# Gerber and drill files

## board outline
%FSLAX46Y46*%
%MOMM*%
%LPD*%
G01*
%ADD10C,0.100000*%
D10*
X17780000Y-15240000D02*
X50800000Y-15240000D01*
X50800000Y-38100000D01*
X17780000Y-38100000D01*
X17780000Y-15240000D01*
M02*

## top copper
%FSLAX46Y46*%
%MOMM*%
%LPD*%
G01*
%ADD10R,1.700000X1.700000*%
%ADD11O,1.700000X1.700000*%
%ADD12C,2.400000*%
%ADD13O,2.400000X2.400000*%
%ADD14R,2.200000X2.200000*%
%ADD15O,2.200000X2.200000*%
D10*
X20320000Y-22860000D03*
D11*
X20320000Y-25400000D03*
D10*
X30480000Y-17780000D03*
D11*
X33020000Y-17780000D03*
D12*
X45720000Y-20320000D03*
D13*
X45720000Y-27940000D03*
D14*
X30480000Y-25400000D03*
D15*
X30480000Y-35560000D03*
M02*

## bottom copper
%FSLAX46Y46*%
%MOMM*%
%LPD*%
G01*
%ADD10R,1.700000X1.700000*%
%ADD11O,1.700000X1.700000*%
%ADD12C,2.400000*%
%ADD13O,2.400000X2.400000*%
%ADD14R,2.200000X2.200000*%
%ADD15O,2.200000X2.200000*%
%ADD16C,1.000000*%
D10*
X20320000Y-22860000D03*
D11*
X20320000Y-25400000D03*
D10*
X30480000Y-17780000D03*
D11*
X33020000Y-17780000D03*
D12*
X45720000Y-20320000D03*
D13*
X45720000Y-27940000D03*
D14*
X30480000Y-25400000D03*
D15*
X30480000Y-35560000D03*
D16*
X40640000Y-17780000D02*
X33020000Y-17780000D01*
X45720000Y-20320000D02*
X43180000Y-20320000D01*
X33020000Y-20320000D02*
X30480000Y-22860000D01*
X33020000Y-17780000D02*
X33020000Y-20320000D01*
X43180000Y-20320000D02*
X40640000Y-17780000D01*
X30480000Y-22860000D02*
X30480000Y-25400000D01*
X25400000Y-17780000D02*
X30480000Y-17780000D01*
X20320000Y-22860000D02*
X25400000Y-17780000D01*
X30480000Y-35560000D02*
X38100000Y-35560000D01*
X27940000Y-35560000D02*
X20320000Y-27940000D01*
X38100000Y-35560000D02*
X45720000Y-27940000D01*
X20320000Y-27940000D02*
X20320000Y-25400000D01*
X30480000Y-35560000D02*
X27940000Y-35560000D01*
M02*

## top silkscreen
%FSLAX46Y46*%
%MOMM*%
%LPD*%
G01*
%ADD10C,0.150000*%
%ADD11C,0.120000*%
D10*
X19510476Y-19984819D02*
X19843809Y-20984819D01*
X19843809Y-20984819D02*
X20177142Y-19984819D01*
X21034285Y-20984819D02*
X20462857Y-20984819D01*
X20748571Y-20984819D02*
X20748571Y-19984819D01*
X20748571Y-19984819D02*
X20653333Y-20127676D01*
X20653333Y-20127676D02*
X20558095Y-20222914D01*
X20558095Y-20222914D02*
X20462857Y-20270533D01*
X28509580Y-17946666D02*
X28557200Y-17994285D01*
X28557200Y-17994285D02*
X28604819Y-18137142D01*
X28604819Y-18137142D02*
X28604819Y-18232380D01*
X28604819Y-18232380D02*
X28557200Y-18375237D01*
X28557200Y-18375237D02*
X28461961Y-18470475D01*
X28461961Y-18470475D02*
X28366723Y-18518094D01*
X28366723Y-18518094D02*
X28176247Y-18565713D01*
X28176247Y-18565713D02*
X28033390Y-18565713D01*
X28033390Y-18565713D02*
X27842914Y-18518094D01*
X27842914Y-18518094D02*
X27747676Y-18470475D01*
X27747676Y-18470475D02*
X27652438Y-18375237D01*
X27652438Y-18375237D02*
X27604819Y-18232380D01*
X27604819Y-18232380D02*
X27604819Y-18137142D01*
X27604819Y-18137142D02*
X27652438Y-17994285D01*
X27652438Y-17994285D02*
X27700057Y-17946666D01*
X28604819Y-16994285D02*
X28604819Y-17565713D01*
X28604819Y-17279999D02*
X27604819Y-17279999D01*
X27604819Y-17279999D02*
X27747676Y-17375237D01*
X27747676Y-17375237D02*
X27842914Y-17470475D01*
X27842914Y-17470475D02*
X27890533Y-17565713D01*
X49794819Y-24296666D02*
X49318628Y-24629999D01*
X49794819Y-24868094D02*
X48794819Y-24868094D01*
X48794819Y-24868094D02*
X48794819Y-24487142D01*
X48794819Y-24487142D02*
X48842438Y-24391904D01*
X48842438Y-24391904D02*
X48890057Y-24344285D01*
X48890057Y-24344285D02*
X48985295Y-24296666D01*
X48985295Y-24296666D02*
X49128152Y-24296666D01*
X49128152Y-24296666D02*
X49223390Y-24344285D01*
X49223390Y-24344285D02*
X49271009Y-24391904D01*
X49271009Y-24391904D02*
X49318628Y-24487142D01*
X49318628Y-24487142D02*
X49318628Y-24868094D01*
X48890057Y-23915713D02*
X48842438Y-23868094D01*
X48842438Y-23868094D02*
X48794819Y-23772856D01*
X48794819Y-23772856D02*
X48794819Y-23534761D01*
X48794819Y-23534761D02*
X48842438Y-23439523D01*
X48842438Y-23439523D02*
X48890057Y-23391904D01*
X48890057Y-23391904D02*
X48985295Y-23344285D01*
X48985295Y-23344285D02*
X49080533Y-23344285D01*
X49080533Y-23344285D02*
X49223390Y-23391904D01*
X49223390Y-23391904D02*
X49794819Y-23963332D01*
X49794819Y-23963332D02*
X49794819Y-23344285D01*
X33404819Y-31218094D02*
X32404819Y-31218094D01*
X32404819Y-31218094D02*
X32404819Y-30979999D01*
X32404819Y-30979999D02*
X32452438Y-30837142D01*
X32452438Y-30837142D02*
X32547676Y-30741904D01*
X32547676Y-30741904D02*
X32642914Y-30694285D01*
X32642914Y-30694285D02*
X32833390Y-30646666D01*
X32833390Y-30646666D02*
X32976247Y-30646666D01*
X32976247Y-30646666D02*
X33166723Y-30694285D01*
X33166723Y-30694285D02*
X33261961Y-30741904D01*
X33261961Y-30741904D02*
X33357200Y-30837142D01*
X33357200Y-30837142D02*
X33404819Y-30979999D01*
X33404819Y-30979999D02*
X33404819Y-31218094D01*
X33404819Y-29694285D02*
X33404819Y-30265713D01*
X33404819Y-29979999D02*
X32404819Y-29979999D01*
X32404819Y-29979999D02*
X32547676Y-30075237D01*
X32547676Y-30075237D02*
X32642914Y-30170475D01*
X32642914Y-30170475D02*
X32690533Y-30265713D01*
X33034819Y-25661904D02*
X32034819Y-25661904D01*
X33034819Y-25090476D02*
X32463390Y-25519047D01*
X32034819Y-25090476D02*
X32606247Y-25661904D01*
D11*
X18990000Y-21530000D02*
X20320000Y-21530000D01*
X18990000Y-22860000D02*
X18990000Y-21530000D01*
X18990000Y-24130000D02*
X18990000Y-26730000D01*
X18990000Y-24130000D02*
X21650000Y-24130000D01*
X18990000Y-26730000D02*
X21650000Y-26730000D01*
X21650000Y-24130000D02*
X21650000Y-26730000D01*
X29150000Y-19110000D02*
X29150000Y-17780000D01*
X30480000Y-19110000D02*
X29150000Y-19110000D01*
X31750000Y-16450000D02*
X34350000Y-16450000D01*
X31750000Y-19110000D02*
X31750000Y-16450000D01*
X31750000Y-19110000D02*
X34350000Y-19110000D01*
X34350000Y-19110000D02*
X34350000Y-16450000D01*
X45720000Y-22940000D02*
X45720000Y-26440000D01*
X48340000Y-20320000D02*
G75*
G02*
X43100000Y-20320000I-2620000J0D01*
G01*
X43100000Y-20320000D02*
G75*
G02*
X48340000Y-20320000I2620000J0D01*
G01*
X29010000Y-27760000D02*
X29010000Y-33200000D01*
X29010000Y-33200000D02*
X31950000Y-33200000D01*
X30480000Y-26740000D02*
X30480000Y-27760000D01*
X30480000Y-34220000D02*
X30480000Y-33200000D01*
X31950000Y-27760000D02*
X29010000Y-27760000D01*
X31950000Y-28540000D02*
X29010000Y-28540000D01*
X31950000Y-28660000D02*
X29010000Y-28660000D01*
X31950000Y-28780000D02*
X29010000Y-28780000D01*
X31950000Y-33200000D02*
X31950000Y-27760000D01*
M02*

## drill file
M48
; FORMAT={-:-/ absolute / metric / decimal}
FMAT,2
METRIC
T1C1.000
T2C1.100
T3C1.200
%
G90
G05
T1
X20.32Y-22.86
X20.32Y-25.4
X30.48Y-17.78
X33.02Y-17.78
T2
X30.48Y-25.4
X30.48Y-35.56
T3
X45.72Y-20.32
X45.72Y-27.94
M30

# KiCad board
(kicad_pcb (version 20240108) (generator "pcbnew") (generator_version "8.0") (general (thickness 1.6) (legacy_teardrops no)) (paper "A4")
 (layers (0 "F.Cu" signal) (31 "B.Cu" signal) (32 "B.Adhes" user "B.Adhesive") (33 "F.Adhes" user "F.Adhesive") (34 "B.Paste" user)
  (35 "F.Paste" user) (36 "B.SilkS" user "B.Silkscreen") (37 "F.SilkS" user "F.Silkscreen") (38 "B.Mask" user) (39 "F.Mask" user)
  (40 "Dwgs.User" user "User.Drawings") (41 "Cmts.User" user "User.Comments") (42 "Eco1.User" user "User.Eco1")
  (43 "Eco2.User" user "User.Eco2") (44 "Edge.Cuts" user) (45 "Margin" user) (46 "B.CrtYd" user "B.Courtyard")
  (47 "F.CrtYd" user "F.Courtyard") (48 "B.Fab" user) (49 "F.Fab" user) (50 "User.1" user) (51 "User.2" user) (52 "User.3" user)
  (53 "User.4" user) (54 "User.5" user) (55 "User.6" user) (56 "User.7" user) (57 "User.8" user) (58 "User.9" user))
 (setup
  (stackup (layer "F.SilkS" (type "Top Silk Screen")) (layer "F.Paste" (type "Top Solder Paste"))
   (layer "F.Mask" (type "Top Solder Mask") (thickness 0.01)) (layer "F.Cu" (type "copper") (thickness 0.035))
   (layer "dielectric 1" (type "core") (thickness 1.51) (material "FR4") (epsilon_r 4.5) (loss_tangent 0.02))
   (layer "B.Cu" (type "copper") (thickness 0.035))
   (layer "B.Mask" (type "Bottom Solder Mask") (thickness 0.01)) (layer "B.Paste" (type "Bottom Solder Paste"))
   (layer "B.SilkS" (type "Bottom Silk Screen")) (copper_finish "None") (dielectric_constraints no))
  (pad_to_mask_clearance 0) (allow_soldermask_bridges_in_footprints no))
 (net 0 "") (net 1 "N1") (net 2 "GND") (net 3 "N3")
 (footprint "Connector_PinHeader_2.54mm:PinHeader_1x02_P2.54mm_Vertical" (layer "F.Cu") (at 20.32 22.86)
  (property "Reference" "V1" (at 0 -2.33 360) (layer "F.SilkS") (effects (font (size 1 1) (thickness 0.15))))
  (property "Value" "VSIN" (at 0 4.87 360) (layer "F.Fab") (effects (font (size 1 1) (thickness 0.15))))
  (fp_line (start -1.33 -1.33) (end 0 -1.33) (stroke (width 0.12) (type solid)) (layer "F.SilkS"))
  (fp_line (start -1.33 0) (end -1.33 -1.33) (stroke (width 0.12) (type solid)) (layer "F.SilkS"))
  (fp_line (start -1.33 1.27) (end -1.33 3.87) (stroke (width 0.12) (type solid)) (layer "F.SilkS"))
  (fp_line (start -1.33 1.27) (end 1.33 1.27) (stroke (width 0.12) (type solid)) (layer "F.SilkS"))
  (fp_line (start -1.33 3.87) (end 1.33 3.87) (stroke (width 0.12) (type solid)) (layer "F.SilkS"))
  (fp_line (start 1.33 1.27) (end 1.33 3.87) (stroke (width 0.12) (type solid)) (layer "F.SilkS"))
  (pad "1" thru_hole rect (at 0 0) (size 1.7 1.7) (drill 1) (layers "*.Cu" "*.Mask") (remove_unused_layers no) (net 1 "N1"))
  (pad "2" thru_hole oval (at 0 2.54) (size 1.7 1.7) (drill 1) (layers "*.Cu" "*.Mask") (remove_unused_layers no) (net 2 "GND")))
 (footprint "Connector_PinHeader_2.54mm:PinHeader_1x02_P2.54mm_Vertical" (layer "F.Cu") (at 30.48 17.78 90)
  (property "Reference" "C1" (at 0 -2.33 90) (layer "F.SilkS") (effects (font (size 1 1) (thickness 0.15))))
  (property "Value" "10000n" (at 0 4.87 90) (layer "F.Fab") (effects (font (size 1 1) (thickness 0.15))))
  (fp_line (start -1.33 -1.33) (end 0 -1.33) (stroke (width 0.12) (type solid)) (layer "F.SilkS"))
  (fp_line (start -1.33 0) (end -1.33 -1.33) (stroke (width 0.12) (type solid)) (layer "F.SilkS"))
  (fp_line (start 1.33 1.27) (end 1.33 3.87) (stroke (width 0.12) (type solid)) (layer "F.SilkS"))
  (fp_line (start -1.33 1.27) (end 1.33 1.27) (stroke (width 0.12) (type solid)) (layer "F.SilkS"))
  (fp_line (start -1.33 1.27) (end -1.33 3.87) (stroke (width 0.12) (type solid)) (layer "F.SilkS"))
  (fp_line (start -1.33 3.87) (end 1.33 3.87) (stroke (width 0.12) (type solid)) (layer "F.SilkS"))
  (pad "1" thru_hole rect (at 0 0 90) (size 1.7 1.7) (drill 1) (layers "*.Cu" "*.Mask") (remove_unused_layers no) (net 1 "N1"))
  (pad "2" thru_hole oval (at 0 2.54 90) (size 1.7 1.7) (drill 1) (layers "*.Cu" "*.Mask") (remove_unused_layers no) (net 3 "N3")))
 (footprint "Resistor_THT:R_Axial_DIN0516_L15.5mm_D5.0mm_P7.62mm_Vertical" (layer "F.Cu") (at 45.72 20.32 -90)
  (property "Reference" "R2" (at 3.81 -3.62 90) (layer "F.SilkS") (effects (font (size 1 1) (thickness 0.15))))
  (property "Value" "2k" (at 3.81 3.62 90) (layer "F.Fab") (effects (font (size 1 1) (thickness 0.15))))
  (fp_line (start 2.62 0) (end 6.12 0) (stroke (width 0.12) (type solid)) (layer "F.SilkS"))
  (fp_circle (center 0 0) (end 2.62 0) (stroke (width 0.12) (type solid)) (fill none) (layer "F.SilkS"))
  (pad "1" thru_hole circle (at 0 0 270) (size 2.4 2.4) (drill 1.2) (layers "*.Cu" "*.Mask") (remove_unused_layers no) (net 3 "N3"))
  (pad "2" thru_hole oval (at 7.62 0 270) (size 2.4 2.4) (drill 1.2) (layers "*.Cu" "*.Mask") (remove_unused_layers no) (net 2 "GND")))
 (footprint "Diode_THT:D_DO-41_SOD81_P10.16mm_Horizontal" (layer "F.Cu") (at 30.48 25.4 -90)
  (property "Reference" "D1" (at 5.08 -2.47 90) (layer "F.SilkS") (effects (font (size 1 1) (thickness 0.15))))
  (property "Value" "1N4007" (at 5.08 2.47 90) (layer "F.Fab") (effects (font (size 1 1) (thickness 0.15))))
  (fp_line (start 2.36 1.47) (end 7.8 1.47) (stroke (width 0.12) (type solid)) (layer "F.SilkS"))
  (fp_line (start 7.8 1.47) (end 7.8 -1.47) (stroke (width 0.12) (type solid)) (layer "F.SilkS"))
  (fp_line (start 1.34 0) (end 2.36 0) (stroke (width 0.12) (type solid)) (layer "F.SilkS"))
  (fp_line (start 8.82 0) (end 7.8 0) (stroke (width 0.12) (type solid)) (layer "F.SilkS"))
  (fp_line (start 2.36 -1.47) (end 2.36 1.47) (stroke (width 0.12) (type solid)) (layer "F.SilkS"))
  (fp_line (start 3.14 -1.47) (end 3.14 1.47) (stroke (width 0.12) (type solid)) (layer "F.SilkS"))
  (fp_line (start 3.26 -1.47) (end 3.26 1.47) (stroke (width 0.12) (type solid)) (layer "F.SilkS"))
  (fp_line (start 3.38 -1.47) (end 3.38 1.47) (stroke (width 0.12) (type solid)) (layer "F.SilkS"))
  (fp_line (start 7.8 -1.47) (end 2.36 -1.47) (stroke (width 0.12) (type solid)) (layer "F.SilkS"))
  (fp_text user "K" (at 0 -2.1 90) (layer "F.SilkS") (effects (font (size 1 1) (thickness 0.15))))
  (pad "1" thru_hole rect (at 0 0 270) (size 2.2 2.2) (drill 1.1) (layers "*.Cu" "*.Mask") (remove_unused_layers no) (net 3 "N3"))
  (pad "2" thru_hole oval (at 10.16 0 270) (size 2.2 2.2) (drill 1.1) (layers "*.Cu" "*.Mask") (remove_unused_layers no) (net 2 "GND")))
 (gr_rect (start 17.78 15.24) (end 50.8 38.1) (stroke (width 0.1) (type default)) (fill none) (layer "Edge.Cuts"))
 (segment (start 40.64 17.78) (end 33.02 17.78) (width 1) (layer "B.Cu") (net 3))
 (segment (start 45.72 20.32) (end 43.18 20.32) (width 1) (layer "B.Cu") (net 3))
 (segment (start 33.02 20.32) (end 30.48 22.86) (width 1) (layer "B.Cu") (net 3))
 (segment (start 33.02 17.78) (end 33.02 20.32) (width 1) (layer "B.Cu") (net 3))
 (segment (start 43.18 20.32) (end 40.64 17.78) (width 1) (layer "B.Cu") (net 3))
 (segment (start 30.48 22.86) (end 30.48 25.4) (width 1) (layer "B.Cu") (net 3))
 (segment (start 25.4 17.78) (end 30.48 17.78) (width 1) (layer "B.Cu") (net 1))
 (segment (start 20.32 22.86) (end 25.4 17.78) (width 1) (layer "B.Cu") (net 1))
 (segment (start 30.48 35.56) (end 38.1 35.56) (width 1) (layer "B.Cu") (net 2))
 (segment (start 27.94 35.56) (end 20.32 27.94) (width 1) (layer "B.Cu") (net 2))
 (segment (start 38.1 35.56) (end 45.72 27.94) (width 1) (layer "B.Cu") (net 2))
 (segment (start 20.32 27.94) (end 20.32 25.4) (width 1) (layer "B.Cu") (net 2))
 (segment (start 30.48 35.56) (end 27.94 35.56) (width 1) (layer "B.Cu") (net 2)))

